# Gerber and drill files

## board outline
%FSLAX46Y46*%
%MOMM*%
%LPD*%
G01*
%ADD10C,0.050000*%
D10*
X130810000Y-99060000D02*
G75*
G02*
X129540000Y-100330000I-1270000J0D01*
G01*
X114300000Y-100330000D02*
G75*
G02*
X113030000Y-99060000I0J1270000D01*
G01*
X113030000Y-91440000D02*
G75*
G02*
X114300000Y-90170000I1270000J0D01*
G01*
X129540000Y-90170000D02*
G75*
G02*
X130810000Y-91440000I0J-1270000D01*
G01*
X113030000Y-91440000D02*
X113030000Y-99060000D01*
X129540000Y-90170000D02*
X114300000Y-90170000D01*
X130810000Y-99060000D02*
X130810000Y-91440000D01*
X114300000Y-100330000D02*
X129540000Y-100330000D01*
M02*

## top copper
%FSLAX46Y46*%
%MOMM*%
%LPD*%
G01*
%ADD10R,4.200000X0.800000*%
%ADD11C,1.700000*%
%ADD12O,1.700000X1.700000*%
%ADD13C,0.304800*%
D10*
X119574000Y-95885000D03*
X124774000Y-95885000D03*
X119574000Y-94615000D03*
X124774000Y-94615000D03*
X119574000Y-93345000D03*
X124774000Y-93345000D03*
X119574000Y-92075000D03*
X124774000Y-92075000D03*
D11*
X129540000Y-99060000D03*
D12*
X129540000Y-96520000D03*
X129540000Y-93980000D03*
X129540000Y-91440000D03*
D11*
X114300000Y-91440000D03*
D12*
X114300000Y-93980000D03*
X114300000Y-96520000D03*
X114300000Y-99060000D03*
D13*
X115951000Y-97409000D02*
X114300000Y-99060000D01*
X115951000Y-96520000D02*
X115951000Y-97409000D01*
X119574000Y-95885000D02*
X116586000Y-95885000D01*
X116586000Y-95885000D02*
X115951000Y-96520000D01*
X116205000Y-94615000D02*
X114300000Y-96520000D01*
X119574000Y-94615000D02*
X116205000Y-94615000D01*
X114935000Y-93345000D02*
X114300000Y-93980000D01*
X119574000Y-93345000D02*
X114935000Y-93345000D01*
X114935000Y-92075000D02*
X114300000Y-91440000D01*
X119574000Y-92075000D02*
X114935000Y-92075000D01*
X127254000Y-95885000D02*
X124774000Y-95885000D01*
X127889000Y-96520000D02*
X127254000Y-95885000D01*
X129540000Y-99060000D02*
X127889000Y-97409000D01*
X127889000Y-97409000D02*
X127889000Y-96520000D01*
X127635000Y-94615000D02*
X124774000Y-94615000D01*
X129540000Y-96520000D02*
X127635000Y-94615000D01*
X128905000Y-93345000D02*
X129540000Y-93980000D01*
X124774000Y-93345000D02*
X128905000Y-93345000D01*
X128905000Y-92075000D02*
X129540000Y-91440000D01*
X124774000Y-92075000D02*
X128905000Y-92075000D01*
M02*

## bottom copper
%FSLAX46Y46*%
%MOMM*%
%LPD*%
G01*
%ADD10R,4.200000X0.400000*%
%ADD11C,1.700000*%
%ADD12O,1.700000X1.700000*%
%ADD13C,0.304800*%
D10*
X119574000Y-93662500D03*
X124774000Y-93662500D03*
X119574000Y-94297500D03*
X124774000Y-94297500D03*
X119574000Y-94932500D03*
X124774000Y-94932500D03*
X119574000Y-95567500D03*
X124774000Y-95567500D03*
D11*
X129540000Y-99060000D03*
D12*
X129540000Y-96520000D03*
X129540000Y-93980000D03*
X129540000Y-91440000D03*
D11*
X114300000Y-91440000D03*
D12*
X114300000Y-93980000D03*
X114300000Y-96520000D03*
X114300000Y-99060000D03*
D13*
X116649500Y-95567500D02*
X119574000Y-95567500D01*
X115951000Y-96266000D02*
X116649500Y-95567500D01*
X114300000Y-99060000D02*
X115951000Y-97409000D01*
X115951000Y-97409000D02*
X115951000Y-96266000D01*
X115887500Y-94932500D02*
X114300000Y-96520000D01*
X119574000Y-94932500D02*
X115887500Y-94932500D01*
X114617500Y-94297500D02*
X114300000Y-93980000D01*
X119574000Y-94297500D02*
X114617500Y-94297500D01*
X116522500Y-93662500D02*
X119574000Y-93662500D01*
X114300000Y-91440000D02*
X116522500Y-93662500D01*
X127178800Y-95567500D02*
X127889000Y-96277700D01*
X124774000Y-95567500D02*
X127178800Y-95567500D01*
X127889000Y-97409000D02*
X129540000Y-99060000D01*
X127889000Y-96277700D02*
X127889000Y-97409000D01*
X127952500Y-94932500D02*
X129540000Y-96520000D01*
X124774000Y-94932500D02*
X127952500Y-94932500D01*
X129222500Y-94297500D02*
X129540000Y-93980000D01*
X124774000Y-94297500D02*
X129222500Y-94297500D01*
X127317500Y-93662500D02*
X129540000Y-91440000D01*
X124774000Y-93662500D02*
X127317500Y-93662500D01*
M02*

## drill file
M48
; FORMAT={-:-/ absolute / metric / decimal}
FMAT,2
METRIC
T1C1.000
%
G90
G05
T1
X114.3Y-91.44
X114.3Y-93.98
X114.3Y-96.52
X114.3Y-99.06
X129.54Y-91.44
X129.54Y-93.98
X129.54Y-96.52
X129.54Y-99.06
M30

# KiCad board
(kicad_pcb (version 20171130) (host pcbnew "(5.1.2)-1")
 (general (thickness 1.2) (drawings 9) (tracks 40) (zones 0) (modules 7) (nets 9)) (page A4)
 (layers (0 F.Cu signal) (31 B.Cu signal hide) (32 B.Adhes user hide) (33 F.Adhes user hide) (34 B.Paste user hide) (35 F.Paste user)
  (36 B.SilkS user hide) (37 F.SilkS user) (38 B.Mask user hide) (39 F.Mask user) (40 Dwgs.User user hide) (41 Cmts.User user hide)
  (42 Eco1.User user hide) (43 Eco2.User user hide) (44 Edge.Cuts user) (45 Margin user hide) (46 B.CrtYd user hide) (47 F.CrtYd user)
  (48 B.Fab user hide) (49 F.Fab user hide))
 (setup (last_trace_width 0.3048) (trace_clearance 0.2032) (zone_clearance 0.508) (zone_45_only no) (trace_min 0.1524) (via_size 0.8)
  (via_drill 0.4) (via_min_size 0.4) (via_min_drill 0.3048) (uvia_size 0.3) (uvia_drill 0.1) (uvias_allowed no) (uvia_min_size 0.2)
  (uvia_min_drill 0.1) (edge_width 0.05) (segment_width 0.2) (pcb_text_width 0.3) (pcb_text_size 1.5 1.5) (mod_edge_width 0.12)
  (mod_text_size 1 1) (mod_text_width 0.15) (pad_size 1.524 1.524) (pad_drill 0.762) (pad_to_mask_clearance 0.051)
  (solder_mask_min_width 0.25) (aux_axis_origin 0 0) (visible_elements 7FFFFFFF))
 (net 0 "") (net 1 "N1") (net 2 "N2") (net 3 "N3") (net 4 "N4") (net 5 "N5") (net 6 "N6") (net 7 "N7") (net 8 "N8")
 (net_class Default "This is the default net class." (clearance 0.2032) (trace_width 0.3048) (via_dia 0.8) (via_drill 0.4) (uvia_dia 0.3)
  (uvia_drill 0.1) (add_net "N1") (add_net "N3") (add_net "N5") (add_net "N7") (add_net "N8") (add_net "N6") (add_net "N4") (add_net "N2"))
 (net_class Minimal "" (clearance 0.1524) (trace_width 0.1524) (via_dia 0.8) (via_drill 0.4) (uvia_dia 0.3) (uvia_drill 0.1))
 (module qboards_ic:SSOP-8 (layer B.Cu) (at 122.174 94.615 90)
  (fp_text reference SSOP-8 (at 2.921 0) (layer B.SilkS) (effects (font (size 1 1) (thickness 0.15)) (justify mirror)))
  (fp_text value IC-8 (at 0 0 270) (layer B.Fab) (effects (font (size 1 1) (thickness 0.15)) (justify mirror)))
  (pad 4 smd rect (at 0.9525 -2.6 90) (size 0.4 4.2) (layers B.Cu B.Paste B.Mask) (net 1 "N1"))
  (pad 5 smd rect (at 0.9525 2.6 90) (size 0.4 4.2) (layers B.Cu B.Paste B.Mask) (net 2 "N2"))
  (pad 3 smd rect (at 0.3175 -2.6 90) (size 0.4 4.2) (layers B.Cu B.Paste B.Mask) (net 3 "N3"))
  (pad 6 smd rect (at 0.3175 2.6 90) (size 0.4 4.2) (layers B.Cu B.Paste B.Mask) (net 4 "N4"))
  (pad 2 smd rect (at -0.3175 -2.6 90) (size 0.4 4.2) (layers B.Cu B.Paste B.Mask) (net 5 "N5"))
  (pad 7 smd rect (at -0.3175 2.6 90) (size 0.4 4.2) (layers B.Cu B.Paste B.Mask) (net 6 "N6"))
  (pad 1 smd rect (at -0.9525 -2.6 90) (size 0.4 4.2) (layers B.Cu B.Paste B.Mask) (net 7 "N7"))
  (pad 8 smd rect (at -0.9525 2.6 90) (size 0.4 4.2) (layers B.Cu B.Paste B.Mask) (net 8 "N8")))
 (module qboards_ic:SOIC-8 (layer F.Cu) (at 122.174 93.98 270)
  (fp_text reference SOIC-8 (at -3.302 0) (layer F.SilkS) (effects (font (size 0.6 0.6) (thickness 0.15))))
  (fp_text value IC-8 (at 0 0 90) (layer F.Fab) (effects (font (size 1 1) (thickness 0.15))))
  (pad 4 smd rect (at 1.905 2.6 270) (size 0.8 4.2) (layers F.Cu F.Paste F.Mask) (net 7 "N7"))
  (pad 5 smd rect (at 1.905 -2.6 270) (size 0.8 4.2) (layers F.Cu F.Paste F.Mask) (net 8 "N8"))
  (pad 3 smd rect (at 0.635 2.6 270) (size 0.8 4.2) (layers F.Cu F.Paste F.Mask) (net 5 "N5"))
  (pad 6 smd rect (at 0.635 -2.6 270) (size 0.8 4.2) (layers F.Cu F.Paste F.Mask) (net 6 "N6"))
  (pad 2 smd rect (at -0.635 2.6 270) (size 0.8 4.2) (layers F.Cu F.Paste F.Mask) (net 3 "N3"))
  (pad 7 smd rect (at -0.635 -2.6 270) (size 0.8 4.2) (layers F.Cu F.Paste F.Mask) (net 4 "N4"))
  (pad 1 smd rect (at -1.905 2.6 270) (size 0.8 4.2) (layers F.Cu F.Paste F.Mask) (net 1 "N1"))
  (pad 8 smd rect (at -1.905 -2.6 270) (size 0.8 4.2) (layers F.Cu F.Paste F.Mask) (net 2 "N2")))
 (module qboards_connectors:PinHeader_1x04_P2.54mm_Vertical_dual (layer F.Cu) (at 129.54 99.06 180)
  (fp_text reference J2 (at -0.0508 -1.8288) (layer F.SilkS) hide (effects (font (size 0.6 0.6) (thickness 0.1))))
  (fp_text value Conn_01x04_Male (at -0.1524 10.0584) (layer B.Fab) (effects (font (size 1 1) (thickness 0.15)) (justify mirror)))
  (pad 1 thru_hole circle (at 0 0 180) (size 1.7 1.7) (drill 1) (layers *.Cu *.Mask) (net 8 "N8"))
  (pad 2 thru_hole oval (at 0 2.54 180) (size 1.7 1.7) (drill 1) (layers *.Cu *.Mask) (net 6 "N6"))
  (pad 3 thru_hole oval (at 0 5.08 180) (size 1.7 1.7) (drill 1) (layers *.Cu *.Mask) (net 4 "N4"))
  (pad 4 thru_hole oval (at 0 7.62 180) (size 1.7 1.7) (drill 1) (layers *.Cu *.Mask) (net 2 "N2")))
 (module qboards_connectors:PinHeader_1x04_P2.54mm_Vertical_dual (layer F.Cu) (at 114.3 91.44)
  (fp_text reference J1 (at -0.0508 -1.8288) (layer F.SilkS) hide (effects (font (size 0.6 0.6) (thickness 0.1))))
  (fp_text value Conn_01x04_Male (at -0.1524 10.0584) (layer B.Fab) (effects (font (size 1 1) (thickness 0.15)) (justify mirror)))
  (pad 1 thru_hole circle (at 0 0) (size 1.7 1.7) (drill 1) (layers *.Cu *.Mask) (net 1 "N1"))
  (pad 2 thru_hole oval (at 0 2.54) (size 1.7 1.7) (drill 1) (layers *.Cu *.Mask) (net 3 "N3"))
  (pad 3 thru_hole oval (at 0 5.08) (size 1.7 1.7) (drill 1) (layers *.Cu *.Mask) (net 5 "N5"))
  (pad 4 thru_hole oval (at 0 7.62) (size 1.7 1.7) (drill 1) (layers *.Cu *.Mask) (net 7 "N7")))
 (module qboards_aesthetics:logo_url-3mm (layer F.Cu) (at 117.602 98.552)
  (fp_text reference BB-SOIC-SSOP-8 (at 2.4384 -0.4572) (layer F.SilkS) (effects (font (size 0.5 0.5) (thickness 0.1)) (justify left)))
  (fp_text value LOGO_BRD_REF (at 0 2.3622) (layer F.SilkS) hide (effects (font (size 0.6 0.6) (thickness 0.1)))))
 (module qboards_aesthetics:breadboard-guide (layer F.Cu) (at 99.06 91.44)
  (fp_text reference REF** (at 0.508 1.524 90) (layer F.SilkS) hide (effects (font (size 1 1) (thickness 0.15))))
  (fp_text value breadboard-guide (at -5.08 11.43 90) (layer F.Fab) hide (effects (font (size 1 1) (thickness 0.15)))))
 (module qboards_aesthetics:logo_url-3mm (layer B.Cu) (at 126.492 98.552 180)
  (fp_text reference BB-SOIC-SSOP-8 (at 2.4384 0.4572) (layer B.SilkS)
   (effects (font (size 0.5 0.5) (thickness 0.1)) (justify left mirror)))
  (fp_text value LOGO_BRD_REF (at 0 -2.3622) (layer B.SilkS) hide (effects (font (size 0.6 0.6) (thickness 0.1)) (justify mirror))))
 (gr_arc (start 129.54 99.06) (end 129.54 100.33) (angle -90) (layer Edge.Cuts) (width 0.05))
 (gr_arc (start 114.3 99.06) (end 113.03 99.06) (angle -90) (layer Edge.Cuts) (width 0.05))
 (gr_arc (start 114.3 91.44) (end 114.3 90.17) (angle -90) (layer Edge.Cuts) (width 0.05))
 (gr_arc (start 129.54 91.44) (end 130.81 91.44) (angle -90) (layer Edge.Cuts) (width 0.05))
 (gr_line (start 113.03 91.44) (end 113.03 99.06) (layer Edge.Cuts) (width 0.05))
 (gr_line (start 129.54 90.17) (end 114.3 90.17) (layer Edge.Cuts) (width 0.05))
 (gr_line (start 130.81 99.06) (end 130.81 91.44) (layer Edge.Cuts) (width 0.05))
 (gr_line (start 114.3 100.33) (end 129.54 100.33) (layer Edge.Cuts) (width 0.05))
 (segment (start 115.951 97.409) (end 114.3 99.06) (width 0.3048) (layer F.Cu) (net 7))
 (segment (start 115.951 96.52) (end 115.951 97.409) (width 0.3048) (layer F.Cu) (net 7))
 (segment (start 119.574 95.885) (end 116.586 95.885) (width 0.3048) (layer F.Cu) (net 7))
 (segment (start 116.586 95.885) (end 115.951 96.52) (width 0.3048) (layer F.Cu) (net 7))
 (segment (start 116.6495 95.5675) (end 119.574 95.5675) (width 0.3048) (layer B.Cu) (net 7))
 (segment (start 115.951 96.266) (end 116.6495 95.5675) (width 0.3048) (layer B.Cu) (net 7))
 (segment (start 114.3 99.06) (end 115.951 97.409) (width 0.3048) (layer B.Cu) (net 7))
 (segment (start 115.951 97.409) (end 115.951 96.266) (width 0.3048) (layer B.Cu) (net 7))
 (segment (start 116.205 94.615) (end 114.3 96.52) (width 0.3048) (layer F.Cu) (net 5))
 (segment (start 119.574 94.615) (end 116.205 94.615) (width 0.3048) (layer F.Cu) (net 5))
 (segment (start 115.8875 94.9325) (end 114.3 96.52) (width 0.3048) (layer B.Cu) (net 5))
 (segment (start 119.574 94.9325) (end 115.8875 94.9325) (width 0.3048) (layer B.Cu) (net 5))
 (segment (start 114.935 93.345) (end 114.3 93.98) (width 0.3048) (layer F.Cu) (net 3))
 (segment (start 119.574 93.345) (end 114.935 93.345) (width 0.3048) (layer F.Cu) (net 3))
 (segment (start 114.6175 94.2975) (end 114.3 93.98) (width 0.3048) (layer B.Cu) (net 3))
 (segment (start 119.574 94.2975) (end 114.6175 94.2975) (width 0.3048) (layer B.Cu) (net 3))
 (segment (start 114.935 92.075) (end 114.3 91.44) (width 0.3048) (layer F.Cu) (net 1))
 (segment (start 119.574 92.075) (end 114.935 92.075) (width 0.3048) (layer F.Cu) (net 1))
 (segment (start 116.5225 93.6625) (end 119.574 93.6625) (width 0.3048) (layer B.Cu) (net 1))
 (segment (start 114.3 91.44) (end 116.5225 93.6625) (width 0.3048) (layer B.Cu) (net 1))
 (segment (start 127.254 95.885) (end 124.774 95.885) (width 0.3048) (layer F.Cu) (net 8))
 (segment (start 127.889 96.52) (end 127.254 95.885) (width 0.3048) (layer F.Cu) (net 8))
 (segment (start 129.54 99.06) (end 127.889 97.409) (width 0.3048) (layer F.Cu) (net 8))
 (segment (start 127.889 97.409) (end 127.889 96.52) (width 0.3048) (layer F.Cu) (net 8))
 (segment (start 127.1788 95.5675) (end 127.889 96.2777) (width 0.3048) (layer B.Cu) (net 8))
 (segment (start 124.774 95.5675) (end 127.1788 95.5675) (width 0.3048) (layer B.Cu) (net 8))
 (segment (start 127.889 97.409) (end 129.54 99.06) (width 0.3048) (layer B.Cu) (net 8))
 (segment (start 127.889 96.2777) (end 127.889 97.409) (width 0.3048) (layer B.Cu) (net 8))
 (segment (start 127.635 94.615) (end 124.774 94.615) (width 0.3048) (layer F.Cu) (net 6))
 (segment (start 129.54 96.52) (end 127.635 94.615) (width 0.3048) (layer F.Cu) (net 6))
 (segment (start 127.9525 94.9325) (end 129.54 96.52) (width 0.3048) (layer B.Cu) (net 6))
 (segment (start 124.774 94.9325) (end 127.9525 94.9325) (width 0.3048) (layer B.Cu) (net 6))
 (segment (start 128.905 93.345) (end 129.54 93.98) (width 0.3048) (layer F.Cu) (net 4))
 (segment (start 124.774 93.345) (end 128.905 93.345) (width 0.3048) (layer F.Cu) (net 4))
 (segment (start 129.2225 94.2975) (end 129.54 93.98) (width 0.3048) (layer B.Cu) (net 4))
 (segment (start 124.774 94.2975) (end 129.2225 94.2975) (width 0.3048) (layer B.Cu) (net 4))
 (segment (start 128.905 92.075) (end 129.54 91.44) (width 0.3048) (layer F.Cu) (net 2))
 (segment (start 124.774 92.075) (end 128.905 92.075) (width 0.3048) (layer F.Cu) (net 2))
 (segment (start 127.3175 93.6625) (end 129.54 91.44) (width 0.3048) (layer B.Cu) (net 2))
 (segment (start 124.774 93.6625) (end 127.3175 93.6625) (width 0.3048) (layer B.Cu) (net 2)))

